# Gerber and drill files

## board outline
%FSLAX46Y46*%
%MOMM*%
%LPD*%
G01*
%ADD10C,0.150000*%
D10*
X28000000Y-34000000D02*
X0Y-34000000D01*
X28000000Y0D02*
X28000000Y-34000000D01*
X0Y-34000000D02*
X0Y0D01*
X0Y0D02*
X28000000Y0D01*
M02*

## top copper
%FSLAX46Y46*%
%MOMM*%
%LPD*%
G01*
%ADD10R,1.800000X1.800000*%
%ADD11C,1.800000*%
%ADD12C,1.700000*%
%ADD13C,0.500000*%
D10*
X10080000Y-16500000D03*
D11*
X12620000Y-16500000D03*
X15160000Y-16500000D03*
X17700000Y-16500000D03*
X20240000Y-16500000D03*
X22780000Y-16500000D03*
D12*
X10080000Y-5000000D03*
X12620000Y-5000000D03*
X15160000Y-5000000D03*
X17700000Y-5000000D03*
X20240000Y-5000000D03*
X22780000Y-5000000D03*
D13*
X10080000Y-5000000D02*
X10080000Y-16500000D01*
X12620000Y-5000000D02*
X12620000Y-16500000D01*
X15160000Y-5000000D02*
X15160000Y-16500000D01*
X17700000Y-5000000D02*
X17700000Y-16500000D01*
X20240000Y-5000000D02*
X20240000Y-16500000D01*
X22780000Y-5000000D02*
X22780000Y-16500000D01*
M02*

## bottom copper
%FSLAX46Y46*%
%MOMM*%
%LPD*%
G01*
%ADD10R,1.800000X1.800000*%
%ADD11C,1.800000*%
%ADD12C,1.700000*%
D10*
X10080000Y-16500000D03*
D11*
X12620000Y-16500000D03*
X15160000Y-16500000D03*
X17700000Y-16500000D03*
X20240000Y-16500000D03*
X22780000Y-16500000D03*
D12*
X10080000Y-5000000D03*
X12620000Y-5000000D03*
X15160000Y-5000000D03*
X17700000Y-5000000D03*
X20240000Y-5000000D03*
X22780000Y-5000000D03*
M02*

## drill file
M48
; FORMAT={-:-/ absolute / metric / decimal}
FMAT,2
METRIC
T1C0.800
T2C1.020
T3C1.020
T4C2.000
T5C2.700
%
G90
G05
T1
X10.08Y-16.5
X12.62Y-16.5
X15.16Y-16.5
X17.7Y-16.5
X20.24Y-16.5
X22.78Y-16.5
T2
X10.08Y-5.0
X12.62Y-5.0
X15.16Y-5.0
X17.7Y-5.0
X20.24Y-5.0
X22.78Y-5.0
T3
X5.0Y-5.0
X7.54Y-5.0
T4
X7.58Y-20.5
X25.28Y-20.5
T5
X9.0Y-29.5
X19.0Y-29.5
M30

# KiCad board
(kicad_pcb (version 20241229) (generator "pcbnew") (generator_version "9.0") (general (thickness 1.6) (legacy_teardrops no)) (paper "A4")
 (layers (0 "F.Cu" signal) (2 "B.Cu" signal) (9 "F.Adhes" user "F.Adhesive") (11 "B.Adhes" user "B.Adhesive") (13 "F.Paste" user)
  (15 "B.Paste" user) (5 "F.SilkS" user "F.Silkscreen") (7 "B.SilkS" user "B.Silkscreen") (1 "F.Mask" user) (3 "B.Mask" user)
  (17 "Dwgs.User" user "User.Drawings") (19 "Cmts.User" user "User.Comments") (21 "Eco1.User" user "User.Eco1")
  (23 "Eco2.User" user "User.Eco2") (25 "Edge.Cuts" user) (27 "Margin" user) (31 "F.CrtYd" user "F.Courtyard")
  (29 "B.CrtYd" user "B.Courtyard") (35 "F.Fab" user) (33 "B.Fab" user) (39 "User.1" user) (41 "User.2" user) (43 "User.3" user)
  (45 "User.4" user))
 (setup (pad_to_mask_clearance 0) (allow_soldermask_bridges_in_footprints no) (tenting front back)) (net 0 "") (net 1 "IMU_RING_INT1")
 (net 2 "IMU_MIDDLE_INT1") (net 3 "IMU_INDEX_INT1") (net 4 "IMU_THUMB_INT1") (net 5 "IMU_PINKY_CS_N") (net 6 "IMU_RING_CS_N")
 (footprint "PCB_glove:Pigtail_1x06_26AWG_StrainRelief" (layer "F.Cu") (at 10.08 16.5)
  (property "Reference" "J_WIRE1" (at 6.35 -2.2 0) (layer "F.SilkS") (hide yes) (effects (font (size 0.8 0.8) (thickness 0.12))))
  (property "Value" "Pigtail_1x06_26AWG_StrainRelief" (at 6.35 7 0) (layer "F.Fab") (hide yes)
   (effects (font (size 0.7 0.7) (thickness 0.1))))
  (pad "" np_thru_hole circle (at -2.5 4) (size 2 2) (drill 2) (layers "*.Cu" "*.Mask"))
  (pad "" np_thru_hole circle (at 15.2 4) (size 2 2) (drill 2) (layers "*.Cu" "*.Mask"))
  (pad "1" thru_hole rect (at 0 0) (size 1.8 1.8) (drill 0.8) (layers "*.Cu" "*.Mask") (remove_unused_layers no) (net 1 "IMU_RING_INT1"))
  (pad "2" thru_hole circle (at 2.54 0) (size 1.8 1.8) (drill 0.8) (layers "*.Cu" "*.Mask") (remove_unused_layers no)
   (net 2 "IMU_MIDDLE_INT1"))
  (pad "3" thru_hole circle (at 5.08 0) (size 1.8 1.8) (drill 0.8) (layers "*.Cu" "*.Mask") (remove_unused_layers no)
   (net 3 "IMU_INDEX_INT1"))
  (pad "4" thru_hole circle (at 7.62 0) (size 1.8 1.8) (drill 0.8) (layers "*.Cu" "*.Mask") (remove_unused_layers no)
   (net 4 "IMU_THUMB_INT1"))
  (pad "5" thru_hole circle (at 10.16 0) (size 1.8 1.8) (drill 0.8) (layers "*.Cu" "*.Mask") (remove_unused_layers no)
   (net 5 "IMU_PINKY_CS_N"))
  (pad "6" thru_hole circle (at 12.7 0) (size 1.8 1.8) (drill 0.8) (layers "*.Cu" "*.Mask") (remove_unused_layers no)
   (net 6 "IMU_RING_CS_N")))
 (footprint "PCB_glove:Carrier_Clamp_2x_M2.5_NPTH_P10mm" (layer "F.Cu") (at 14 29.5)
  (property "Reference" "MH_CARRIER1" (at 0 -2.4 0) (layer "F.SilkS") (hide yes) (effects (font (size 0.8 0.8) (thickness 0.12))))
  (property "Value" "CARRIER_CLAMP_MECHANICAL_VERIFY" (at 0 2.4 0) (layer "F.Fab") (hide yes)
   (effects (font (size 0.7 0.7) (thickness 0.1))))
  (pad "" np_thru_hole circle (at -5 0) (size 2.7 2.7) (drill 2.7) (layers "*.Cu" "*.Mask"))
  (pad "" np_thru_hole circle (at 5 0) (size 2.7 2.7) (drill 2.7) (layers "*.Cu" "*.Mask")))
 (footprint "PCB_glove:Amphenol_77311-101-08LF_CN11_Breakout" (layer "F.Cu") (at 5 5)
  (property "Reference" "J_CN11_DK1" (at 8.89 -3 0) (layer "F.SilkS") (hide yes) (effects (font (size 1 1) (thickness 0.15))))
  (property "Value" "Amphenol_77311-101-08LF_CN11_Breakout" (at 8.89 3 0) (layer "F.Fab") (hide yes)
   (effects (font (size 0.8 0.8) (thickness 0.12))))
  (pad "" np_thru_hole circle (at 0 0) (size 1.02 1.02) (drill 1.02) (layers "*.Cu" "*.Mask"))
  (pad "" np_thru_hole circle (at 2.54 0) (size 1.02 1.02) (drill 1.02) (layers "*.Cu" "*.Mask"))
  (pad "3" thru_hole circle (at 5.08 0) (size 1.7 1.7) (drill 1.02) (layers "*.Cu" "*.Mask") (remove_unused_layers no)
   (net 1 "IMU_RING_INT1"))
  (pad "4" thru_hole circle (at 7.62 0) (size 1.7 1.7) (drill 1.02) (layers "*.Cu" "*.Mask") (remove_unused_layers no)
   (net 2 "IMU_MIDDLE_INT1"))
  (pad "5" thru_hole circle (at 10.16 0) (size 1.7 1.7) (drill 1.02) (layers "*.Cu" "*.Mask") (remove_unused_layers no)
   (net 3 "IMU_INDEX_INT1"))
  (pad "6" thru_hole circle (at 12.7 0) (size 1.7 1.7) (drill 1.02) (layers "*.Cu" "*.Mask") (remove_unused_layers no)
   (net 4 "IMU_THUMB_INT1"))
  (pad "7" thru_hole circle (at 15.24 0) (size 1.7 1.7) (drill 1.02) (layers "*.Cu" "*.Mask") (remove_unused_layers no)
   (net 5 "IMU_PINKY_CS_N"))
  (pad "8" thru_hole circle (at 17.78 0) (size 1.7 1.7) (drill 1.02) (layers "*.Cu" "*.Mask") (remove_unused_layers no)
   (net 6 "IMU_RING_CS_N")))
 (gr_line (start 28 34) (end 0 34) (stroke (width 0.15) (type default)) (layer "Edge.Cuts"))
 (gr_line (start 28 0) (end 28 34) (stroke (width 0.15) (type default)) (layer "Edge.Cuts"))
 (gr_line (start 0 34) (end 0 0) (stroke (width 0.15) (type default)) (layer "Edge.Cuts"))
 (gr_line (start 0 0) (end 28 0) (stroke (width 0.15) (type default)) (layer "Edge.Cuts"))
 (segment (start 10.08 5) (end 10.08 16.5) (width 0.5) (layer "F.Cu") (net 1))
 (segment (start 12.62 5) (end 12.62 16.5) (width 0.5) (layer "F.Cu") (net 2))
 (segment (start 15.16 5) (end 15.16 16.5) (width 0.5) (layer "F.Cu") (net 3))
 (segment (start 17.7 5) (end 17.7 16.5) (width 0.5) (layer "F.Cu") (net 4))
 (segment (start 20.24 5) (end 20.24 16.5) (width 0.5) (layer "F.Cu") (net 5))
 (segment (start 22.78 5) (end 22.78 16.5) (width 0.5) (layer "F.Cu") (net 6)))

